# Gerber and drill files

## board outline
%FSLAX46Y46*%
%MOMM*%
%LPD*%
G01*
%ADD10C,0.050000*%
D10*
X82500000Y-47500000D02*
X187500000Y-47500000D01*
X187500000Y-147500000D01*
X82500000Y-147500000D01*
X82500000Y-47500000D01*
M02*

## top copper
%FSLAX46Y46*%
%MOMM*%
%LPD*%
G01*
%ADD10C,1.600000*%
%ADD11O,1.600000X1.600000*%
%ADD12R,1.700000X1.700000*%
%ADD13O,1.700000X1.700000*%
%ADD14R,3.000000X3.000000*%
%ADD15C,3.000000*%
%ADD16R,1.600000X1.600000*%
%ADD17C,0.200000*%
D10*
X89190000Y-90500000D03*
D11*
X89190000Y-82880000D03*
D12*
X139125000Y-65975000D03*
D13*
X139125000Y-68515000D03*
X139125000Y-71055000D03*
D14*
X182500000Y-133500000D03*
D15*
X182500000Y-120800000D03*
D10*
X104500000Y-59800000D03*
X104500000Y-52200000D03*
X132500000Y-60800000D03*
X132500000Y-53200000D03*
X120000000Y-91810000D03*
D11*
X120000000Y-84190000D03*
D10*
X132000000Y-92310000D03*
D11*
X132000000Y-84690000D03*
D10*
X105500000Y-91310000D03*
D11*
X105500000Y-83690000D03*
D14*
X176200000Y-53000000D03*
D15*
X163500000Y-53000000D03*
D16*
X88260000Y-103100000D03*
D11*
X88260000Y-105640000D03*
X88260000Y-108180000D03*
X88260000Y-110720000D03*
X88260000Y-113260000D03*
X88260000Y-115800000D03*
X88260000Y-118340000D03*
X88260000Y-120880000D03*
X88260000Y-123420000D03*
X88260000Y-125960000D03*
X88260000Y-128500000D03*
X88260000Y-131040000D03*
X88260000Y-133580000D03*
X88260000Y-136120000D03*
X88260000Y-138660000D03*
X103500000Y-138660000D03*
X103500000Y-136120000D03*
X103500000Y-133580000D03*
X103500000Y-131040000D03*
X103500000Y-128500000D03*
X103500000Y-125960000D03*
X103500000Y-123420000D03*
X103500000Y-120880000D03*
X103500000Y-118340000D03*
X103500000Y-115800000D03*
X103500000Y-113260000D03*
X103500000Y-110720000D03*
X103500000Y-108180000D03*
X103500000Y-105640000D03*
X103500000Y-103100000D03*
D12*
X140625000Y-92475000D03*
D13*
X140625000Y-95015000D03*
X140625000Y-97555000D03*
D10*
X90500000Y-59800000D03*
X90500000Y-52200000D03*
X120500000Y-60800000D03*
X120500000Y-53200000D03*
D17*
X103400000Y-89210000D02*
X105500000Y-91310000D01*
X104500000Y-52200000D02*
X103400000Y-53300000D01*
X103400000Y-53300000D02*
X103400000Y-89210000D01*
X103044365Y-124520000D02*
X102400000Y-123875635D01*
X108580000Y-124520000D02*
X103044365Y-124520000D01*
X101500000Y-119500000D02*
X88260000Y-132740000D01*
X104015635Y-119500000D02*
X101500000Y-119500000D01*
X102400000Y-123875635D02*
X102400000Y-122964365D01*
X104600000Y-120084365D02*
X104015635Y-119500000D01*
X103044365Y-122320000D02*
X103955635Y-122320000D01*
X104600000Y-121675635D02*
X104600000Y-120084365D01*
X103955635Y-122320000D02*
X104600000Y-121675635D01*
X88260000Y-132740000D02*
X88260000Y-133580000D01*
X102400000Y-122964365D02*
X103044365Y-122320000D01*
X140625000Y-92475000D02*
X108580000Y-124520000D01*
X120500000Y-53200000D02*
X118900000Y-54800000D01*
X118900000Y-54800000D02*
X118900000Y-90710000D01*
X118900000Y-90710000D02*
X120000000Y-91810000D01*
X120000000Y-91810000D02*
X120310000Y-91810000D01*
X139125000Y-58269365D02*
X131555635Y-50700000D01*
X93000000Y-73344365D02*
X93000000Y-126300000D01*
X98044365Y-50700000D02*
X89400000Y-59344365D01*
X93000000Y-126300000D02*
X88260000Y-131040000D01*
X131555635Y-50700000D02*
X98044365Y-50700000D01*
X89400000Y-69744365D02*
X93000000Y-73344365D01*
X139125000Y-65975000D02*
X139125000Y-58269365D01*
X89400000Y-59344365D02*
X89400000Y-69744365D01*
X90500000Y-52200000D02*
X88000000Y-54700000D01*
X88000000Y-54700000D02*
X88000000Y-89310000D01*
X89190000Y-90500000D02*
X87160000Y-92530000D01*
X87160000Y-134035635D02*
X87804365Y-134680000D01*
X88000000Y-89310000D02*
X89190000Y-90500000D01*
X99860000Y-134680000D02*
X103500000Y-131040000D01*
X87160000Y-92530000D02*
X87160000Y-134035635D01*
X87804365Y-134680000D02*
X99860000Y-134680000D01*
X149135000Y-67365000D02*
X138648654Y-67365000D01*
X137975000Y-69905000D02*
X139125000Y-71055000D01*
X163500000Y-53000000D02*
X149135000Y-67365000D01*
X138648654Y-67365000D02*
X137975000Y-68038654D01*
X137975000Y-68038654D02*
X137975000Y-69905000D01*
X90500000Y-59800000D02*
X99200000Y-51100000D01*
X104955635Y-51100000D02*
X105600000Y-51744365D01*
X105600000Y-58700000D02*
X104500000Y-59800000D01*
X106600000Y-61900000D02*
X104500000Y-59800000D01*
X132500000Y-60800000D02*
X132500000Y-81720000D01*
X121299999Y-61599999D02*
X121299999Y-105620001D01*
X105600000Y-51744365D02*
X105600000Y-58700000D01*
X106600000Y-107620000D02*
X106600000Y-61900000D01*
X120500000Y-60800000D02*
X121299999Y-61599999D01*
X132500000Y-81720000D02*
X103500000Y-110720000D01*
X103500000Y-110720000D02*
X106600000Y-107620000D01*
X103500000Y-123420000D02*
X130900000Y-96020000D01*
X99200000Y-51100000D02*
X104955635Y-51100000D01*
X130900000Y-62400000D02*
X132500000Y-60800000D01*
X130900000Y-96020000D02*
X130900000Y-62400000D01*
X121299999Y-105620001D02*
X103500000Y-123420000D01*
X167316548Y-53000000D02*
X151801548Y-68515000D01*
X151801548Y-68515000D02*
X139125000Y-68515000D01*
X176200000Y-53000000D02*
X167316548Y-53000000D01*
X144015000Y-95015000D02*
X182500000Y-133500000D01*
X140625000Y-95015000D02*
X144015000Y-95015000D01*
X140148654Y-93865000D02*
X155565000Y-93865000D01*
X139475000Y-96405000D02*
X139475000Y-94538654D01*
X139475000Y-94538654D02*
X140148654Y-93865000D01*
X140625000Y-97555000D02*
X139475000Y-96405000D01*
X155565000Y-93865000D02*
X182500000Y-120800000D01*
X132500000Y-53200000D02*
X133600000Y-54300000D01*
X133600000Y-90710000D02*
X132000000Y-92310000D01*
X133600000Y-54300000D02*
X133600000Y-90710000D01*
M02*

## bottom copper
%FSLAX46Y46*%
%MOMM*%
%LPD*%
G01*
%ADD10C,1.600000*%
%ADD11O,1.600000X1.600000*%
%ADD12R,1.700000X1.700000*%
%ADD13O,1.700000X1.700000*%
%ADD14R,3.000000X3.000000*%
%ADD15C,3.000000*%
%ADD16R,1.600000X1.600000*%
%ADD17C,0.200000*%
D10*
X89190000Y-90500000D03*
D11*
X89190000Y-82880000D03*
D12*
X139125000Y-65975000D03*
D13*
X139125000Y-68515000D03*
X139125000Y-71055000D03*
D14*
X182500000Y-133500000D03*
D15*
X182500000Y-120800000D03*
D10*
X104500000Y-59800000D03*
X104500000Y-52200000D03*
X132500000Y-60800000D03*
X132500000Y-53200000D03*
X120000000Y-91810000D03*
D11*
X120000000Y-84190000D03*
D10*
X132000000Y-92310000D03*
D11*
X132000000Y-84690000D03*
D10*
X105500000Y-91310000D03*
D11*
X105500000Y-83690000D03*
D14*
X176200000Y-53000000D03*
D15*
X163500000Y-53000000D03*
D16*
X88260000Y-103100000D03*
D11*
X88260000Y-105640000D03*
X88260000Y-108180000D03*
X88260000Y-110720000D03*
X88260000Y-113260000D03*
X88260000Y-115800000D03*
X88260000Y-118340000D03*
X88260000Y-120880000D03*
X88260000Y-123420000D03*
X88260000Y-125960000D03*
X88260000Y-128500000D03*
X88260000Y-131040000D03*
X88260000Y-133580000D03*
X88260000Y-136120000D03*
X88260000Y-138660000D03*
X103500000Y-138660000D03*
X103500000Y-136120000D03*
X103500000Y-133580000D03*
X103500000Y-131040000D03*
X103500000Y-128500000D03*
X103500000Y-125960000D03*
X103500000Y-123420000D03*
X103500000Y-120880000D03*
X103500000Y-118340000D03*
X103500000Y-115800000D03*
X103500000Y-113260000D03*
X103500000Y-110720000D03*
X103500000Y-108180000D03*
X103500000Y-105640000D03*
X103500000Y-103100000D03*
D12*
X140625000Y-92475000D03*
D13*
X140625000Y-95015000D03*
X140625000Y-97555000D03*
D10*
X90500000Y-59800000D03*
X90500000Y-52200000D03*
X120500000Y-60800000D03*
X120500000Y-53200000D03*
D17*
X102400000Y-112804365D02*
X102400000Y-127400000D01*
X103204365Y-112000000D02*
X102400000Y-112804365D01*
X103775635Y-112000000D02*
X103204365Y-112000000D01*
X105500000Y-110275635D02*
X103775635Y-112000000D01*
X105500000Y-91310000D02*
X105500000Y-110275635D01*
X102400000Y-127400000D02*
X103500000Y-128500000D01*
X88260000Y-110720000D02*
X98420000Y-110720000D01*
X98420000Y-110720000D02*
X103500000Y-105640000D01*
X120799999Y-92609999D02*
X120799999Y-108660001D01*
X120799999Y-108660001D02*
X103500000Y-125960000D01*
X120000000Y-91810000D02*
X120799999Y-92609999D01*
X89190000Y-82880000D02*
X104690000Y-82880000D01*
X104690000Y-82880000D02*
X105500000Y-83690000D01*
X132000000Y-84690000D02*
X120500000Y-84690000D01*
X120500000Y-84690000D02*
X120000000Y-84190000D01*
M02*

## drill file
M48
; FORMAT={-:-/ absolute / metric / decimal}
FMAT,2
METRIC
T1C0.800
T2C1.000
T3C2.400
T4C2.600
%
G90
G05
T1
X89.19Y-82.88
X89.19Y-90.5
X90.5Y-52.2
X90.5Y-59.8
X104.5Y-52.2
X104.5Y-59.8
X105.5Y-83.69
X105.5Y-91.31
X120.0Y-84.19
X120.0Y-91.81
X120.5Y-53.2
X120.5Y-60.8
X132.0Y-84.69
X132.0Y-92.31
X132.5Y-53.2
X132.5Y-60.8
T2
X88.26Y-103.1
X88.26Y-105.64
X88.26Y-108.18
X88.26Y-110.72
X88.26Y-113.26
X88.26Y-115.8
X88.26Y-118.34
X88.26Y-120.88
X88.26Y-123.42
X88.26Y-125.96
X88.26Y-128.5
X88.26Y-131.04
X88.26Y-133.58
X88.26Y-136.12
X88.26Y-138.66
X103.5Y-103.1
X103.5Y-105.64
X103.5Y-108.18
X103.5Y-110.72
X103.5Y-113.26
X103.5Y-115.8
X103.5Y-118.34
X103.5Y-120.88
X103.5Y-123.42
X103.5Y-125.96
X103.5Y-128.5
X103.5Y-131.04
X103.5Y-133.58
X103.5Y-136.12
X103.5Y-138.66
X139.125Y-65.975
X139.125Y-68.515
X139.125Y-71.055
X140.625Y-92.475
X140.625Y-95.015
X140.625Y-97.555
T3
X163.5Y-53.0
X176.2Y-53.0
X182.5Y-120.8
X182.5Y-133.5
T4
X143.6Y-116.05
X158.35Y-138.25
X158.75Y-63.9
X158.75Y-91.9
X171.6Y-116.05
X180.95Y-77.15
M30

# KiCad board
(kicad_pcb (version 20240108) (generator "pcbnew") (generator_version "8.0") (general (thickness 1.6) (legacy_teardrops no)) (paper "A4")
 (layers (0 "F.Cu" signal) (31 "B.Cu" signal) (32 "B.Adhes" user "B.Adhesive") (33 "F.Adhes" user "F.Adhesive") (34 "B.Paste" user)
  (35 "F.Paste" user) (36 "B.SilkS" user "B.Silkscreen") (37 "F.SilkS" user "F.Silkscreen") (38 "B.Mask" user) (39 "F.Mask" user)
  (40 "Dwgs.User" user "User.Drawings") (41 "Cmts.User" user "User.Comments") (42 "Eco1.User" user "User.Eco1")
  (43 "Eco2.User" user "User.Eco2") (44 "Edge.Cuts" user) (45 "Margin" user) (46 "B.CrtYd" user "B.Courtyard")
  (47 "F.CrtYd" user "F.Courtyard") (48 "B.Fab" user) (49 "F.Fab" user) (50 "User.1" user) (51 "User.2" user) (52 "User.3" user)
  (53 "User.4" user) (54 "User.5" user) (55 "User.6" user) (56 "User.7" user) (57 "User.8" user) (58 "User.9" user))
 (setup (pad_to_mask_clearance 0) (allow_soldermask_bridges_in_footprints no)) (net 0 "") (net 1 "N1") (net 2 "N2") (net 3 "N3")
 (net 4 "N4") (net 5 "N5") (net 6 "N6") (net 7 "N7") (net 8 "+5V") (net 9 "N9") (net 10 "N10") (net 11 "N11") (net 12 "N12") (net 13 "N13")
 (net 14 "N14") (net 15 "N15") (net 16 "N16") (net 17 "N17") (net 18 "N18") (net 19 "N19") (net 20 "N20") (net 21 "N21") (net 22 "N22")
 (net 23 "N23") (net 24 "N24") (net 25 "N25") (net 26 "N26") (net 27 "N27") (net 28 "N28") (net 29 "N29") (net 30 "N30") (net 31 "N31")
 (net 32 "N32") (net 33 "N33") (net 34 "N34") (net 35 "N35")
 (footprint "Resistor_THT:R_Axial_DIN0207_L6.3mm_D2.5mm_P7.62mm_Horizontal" (layer "F.Cu") (at 89.19 90.5 90)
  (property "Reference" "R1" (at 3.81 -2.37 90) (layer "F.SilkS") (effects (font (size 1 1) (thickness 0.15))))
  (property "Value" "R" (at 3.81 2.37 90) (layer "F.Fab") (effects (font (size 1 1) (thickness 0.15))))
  (pad "1" thru_hole circle (at 0 0 90) (size 1.6 1.6) (drill 0.8) (layers "*.Cu" "*.Mask") (remove_unused_layers no) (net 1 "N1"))
  (pad "2" thru_hole oval (at 7.62 0 90) (size 1.6 1.6) (drill 0.8) (layers "*.Cu" "*.Mask") (remove_unused_layers no) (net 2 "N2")))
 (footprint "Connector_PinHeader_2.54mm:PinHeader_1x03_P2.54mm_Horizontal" (layer "F.Cu") (at 139.125 65.975)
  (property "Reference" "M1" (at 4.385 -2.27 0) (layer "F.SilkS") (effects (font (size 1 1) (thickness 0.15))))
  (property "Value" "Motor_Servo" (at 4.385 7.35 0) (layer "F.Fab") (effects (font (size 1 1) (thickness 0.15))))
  (pad "1" thru_hole rect (at 0 0) (size 1.7 1.7) (drill 1) (layers "*.Cu" "*.Mask") (remove_unused_layers no) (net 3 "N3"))
  (pad "2" thru_hole oval (at 0 2.54) (size 1.7 1.7) (drill 1) (layers "*.Cu" "*.Mask") (remove_unused_layers no) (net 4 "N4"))
  (pad "3" thru_hole oval (at 0 5.08) (size 1.7 1.7) (drill 1) (layers "*.Cu" "*.Mask") (remove_unused_layers no) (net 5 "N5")))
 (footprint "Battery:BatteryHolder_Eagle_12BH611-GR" (layer "F.Cu") (at 182.5 133.5)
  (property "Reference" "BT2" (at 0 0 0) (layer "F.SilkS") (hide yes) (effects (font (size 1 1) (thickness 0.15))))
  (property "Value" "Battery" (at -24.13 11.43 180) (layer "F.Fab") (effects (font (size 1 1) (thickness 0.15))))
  (pad "" np_thru_hole circle (at -38.9 -17.45) (size 2.6 2.6) (drill 2.6) (layers "*.Cu" "*.Mask"))
  (pad "" np_thru_hole circle (at -24.15 4.75) (size 2.6 2.6) (drill 2.6) (layers "*.Cu" "*.Mask"))
  (pad "" np_thru_hole circle (at -10.9 -17.45) (size 2.6 2.6) (drill 2.6) (layers "*.Cu" "*.Mask"))
  (pad "1" thru_hole rect (at 0 0) (size 3 3) (drill 2.4) (layers "*.Cu" "*.Mask") (remove_unused_layers no) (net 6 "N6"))
  (pad "2" thru_hole circle (at 0 -12.7) (size 3 3) (drill 2.4) (layers "*.Cu" "*.Mask") (remove_unused_layers no) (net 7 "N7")))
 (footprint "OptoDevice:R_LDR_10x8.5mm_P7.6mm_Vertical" (layer "F.Cu") (at 104.5 59.8 90)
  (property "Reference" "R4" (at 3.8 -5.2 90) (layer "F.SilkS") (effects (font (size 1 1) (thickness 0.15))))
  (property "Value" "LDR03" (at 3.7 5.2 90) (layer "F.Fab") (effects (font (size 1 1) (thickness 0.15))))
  (pad "1" thru_hole circle (at 0 0 90) (size 1.6 1.6) (drill 0.8) (layers "*.Cu" "*.Mask") (remove_unused_layers no) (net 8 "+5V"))
  (pad "2" thru_hole circle (at 7.6 0 90) (size 1.6 1.6) (drill 0.8) (layers "*.Cu" "*.Mask") (remove_unused_layers no) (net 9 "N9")))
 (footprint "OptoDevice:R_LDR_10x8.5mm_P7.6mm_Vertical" (layer "F.Cu") (at 132.5 60.8 90)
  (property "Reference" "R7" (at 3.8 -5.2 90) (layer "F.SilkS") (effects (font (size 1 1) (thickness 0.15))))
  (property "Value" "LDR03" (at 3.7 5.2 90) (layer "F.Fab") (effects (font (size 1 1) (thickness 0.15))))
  (pad "1" thru_hole circle (at 0 0 90) (size 1.6 1.6) (drill 0.8) (layers "*.Cu" "*.Mask") (remove_unused_layers no) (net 8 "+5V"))
  (pad "2" thru_hole circle (at 7.6 0 90) (size 1.6 1.6) (drill 0.8) (layers "*.Cu" "*.Mask") (remove_unused_layers no) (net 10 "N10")))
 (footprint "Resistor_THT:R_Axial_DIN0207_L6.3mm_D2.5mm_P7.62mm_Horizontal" (layer "F.Cu") (at 120 91.81 90)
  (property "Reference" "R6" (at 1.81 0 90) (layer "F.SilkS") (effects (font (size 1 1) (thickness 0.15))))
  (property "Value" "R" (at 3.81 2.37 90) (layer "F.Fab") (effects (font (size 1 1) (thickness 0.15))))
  (pad "1" thru_hole circle (at 0 0 90) (size 1.6 1.6) (drill 0.8) (layers "*.Cu" "*.Mask") (remove_unused_layers no) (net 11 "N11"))
  (pad "2" thru_hole oval (at 7.62 0 90) (size 1.6 1.6) (drill 0.8) (layers "*.Cu" "*.Mask") (remove_unused_layers no) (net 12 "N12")))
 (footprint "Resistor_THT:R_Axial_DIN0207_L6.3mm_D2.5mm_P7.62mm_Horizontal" (layer "F.Cu") (at 132 92.31 90)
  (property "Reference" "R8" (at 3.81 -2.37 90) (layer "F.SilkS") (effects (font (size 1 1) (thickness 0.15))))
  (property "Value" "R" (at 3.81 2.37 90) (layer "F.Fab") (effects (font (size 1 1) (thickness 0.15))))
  (pad "1" thru_hole circle (at 0 0 90) (size 1.6 1.6) (drill 0.8) (layers "*.Cu" "*.Mask") (remove_unused_layers no) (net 10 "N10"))
  (pad "2" thru_hole oval (at 7.62 0 90) (size 1.6 1.6) (drill 0.8) (layers "*.Cu" "*.Mask") (remove_unused_layers no) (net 12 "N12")))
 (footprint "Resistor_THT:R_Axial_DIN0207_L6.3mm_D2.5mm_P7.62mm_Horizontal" (layer "F.Cu") (at 105.5 91.31 90)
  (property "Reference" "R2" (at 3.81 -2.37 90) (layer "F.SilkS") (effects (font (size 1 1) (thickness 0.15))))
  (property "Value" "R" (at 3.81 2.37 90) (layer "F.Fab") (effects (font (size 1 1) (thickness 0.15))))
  (pad "1" thru_hole circle (at 0 0 90) (size 1.6 1.6) (drill 0.8) (layers "*.Cu" "*.Mask") (remove_unused_layers no) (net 9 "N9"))
  (pad "2" thru_hole oval (at 7.62 0 90) (size 1.6 1.6) (drill 0.8) (layers "*.Cu" "*.Mask") (remove_unused_layers no) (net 2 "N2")))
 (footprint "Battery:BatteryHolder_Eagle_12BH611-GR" (layer "F.Cu") (at 176.2 53 90)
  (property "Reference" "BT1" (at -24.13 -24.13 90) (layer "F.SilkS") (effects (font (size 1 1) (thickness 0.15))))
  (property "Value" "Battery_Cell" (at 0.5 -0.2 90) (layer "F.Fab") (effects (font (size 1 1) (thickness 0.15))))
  (pad "" np_thru_hole circle (at -38.9 -17.45 90) (size 2.6 2.6) (drill 2.6) (layers "*.Cu" "*.Mask"))
  (pad "" np_thru_hole circle (at -24.15 4.75 90) (size 2.6 2.6) (drill 2.6) (layers "*.Cu" "*.Mask"))
  (pad "" np_thru_hole circle (at -10.9 -17.45 90) (size 2.6 2.6) (drill 2.6) (layers "*.Cu" "*.Mask"))
  (pad "1" thru_hole rect (at 0 0 90) (size 3 3) (drill 2.4) (layers "*.Cu" "*.Mask") (remove_unused_layers no) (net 4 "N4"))
  (pad "2" thru_hole circle (at 0 -12.7 90) (size 3 3) (drill 2.4) (layers "*.Cu" "*.Mask") (remove_unused_layers no) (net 5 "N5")))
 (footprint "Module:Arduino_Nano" (layer "F.Cu") (at 88.26 103.1)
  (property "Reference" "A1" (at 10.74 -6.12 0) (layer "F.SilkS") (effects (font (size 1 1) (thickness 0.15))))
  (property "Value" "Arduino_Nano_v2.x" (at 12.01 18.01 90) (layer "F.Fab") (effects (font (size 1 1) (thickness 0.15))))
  (pad "1" thru_hole rect (at 0 0) (size 1.6 1.6) (drill 1) (layers "*.Cu" "*.Mask") (remove_unused_layers no) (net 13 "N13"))
  (pad "2" thru_hole oval (at 0 2.54) (size 1.6 1.6) (drill 1) (layers "*.Cu" "*.Mask") (remove_unused_layers no) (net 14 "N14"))
  (pad "3" thru_hole oval (at 0 5.08) (size 1.6 1.6) (drill 1) (layers "*.Cu" "*.Mask") (remove_unused_layers no) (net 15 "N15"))
  (pad "4" thru_hole oval (at 0 7.62) (size 1.6 1.6) (drill 1) (layers "*.Cu" "*.Mask") (remove_unused_layers no) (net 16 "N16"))
  (pad "5" thru_hole oval (at 0 10.16) (size 1.6 1.6) (drill 1) (layers "*.Cu" "*.Mask") (remove_unused_layers no) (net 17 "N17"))
  (pad "6" thru_hole oval (at 0 12.7) (size 1.6 1.6) (drill 1) (layers "*.Cu" "*.Mask") (remove_unused_layers no) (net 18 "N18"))
  (pad "7" thru_hole oval (at 0 15.24) (size 1.6 1.6) (drill 1) (layers "*.Cu" "*.Mask") (remove_unused_layers no) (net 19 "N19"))
  (pad "8" thru_hole oval (at 0 17.78) (size 1.6 1.6) (drill 1) (layers "*.Cu" "*.Mask") (remove_unused_layers no) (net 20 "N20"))
  (pad "9" thru_hole oval (at 0 20.32) (size 1.6 1.6) (drill 1) (layers "*.Cu" "*.Mask") (remove_unused_layers no) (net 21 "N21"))
  (pad "10" thru_hole oval (at 0 22.86) (size 1.6 1.6) (drill 1) (layers "*.Cu" "*.Mask") (remove_unused_layers no) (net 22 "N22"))
  (pad "11" thru_hole oval (at 0 25.4) (size 1.6 1.6) (drill 1) (layers "*.Cu" "*.Mask") (remove_unused_layers no) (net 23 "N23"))
  (pad "12" thru_hole oval (at 0 27.94) (size 1.6 1.6) (drill 1) (layers "*.Cu" "*.Mask") (remove_unused_layers no) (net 3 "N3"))
  (pad "13" thru_hole oval (at 0 30.48) (size 1.6 1.6) (drill 1) (layers "*.Cu" "*.Mask") (remove_unused_layers no) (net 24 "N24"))
  (pad "14" thru_hole oval (at 0 33.02) (size 1.6 1.6) (drill 1) (layers "*.Cu" "*.Mask") (remove_unused_layers no) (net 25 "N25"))
  (pad "15" thru_hole oval (at 0 35.56) (size 1.6 1.6) (drill 1) (layers "*.Cu" "*.Mask") (remove_unused_layers no) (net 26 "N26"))
  (pad "16" thru_hole oval (at 15.24 35.56) (size 1.6 1.6) (drill 1) (layers "*.Cu" "*.Mask") (remove_unused_layers no) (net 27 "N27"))
  (pad "17" thru_hole oval (at 15.24 33.02) (size 1.6 1.6) (drill 1) (layers "*.Cu" "*.Mask") (remove_unused_layers no) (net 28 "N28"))
  (pad "18" thru_hole oval (at 15.24 30.48) (size 1.6 1.6) (drill 1) (layers "*.Cu" "*.Mask") (remove_unused_layers no) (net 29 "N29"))
  (pad "19" thru_hole oval (at 15.24 27.94) (size 1.6 1.6) (drill 1) (layers "*.Cu" "*.Mask") (remove_unused_layers no) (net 1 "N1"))
  (pad "20" thru_hole oval (at 15.24 25.4) (size 1.6 1.6) (drill 1) (layers "*.Cu" "*.Mask") (remove_unused_layers no) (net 9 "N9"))
  (pad "21" thru_hole oval (at 15.24 22.86) (size 1.6 1.6) (drill 1) (layers "*.Cu" "*.Mask") (remove_unused_layers no) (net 11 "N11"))
  (pad "22" thru_hole oval (at 15.24 20.32) (size 1.6 1.6) (drill 1) (layers "*.Cu" "*.Mask") (remove_unused_layers no) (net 8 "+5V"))
  (pad "23" thru_hole oval (at 15.24 17.78) (size 1.6 1.6) (drill 1) (layers "*.Cu" "*.Mask") (remove_unused_layers no) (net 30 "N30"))
  (pad "24" thru_hole oval (at 15.24 15.24) (size 1.6 1.6) (drill 1) (layers "*.Cu" "*.Mask") (remove_unused_layers no) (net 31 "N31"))
  (pad "25" thru_hole oval (at 15.24 12.7) (size 1.6 1.6) (drill 1) (layers "*.Cu" "*.Mask") (remove_unused_layers no) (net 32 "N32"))
  (pad "26" thru_hole oval (at 15.24 10.16) (size 1.6 1.6) (drill 1) (layers "*.Cu" "*.Mask") (remove_unused_layers no) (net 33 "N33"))
  (pad "27" thru_hole oval (at 15.24 7.62) (size 1.6 1.6) (drill 1) (layers "*.Cu" "*.Mask") (remove_unused_layers no) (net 8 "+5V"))
  (pad "28" thru_hole oval (at 15.24 5.08) (size 1.6 1.6) (drill 1) (layers "*.Cu" "*.Mask") (remove_unused_layers no) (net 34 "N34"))
  (pad "29" thru_hole oval (at 15.24 2.54) (size 1.6 1.6) (drill 1) (layers "*.Cu" "*.Mask") (remove_unused_layers no) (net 16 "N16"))
  (pad "30" thru_hole oval (at 15.24 0) (size 1.6 1.6) (drill 1) (layers "*.Cu" "*.Mask") (remove_unused_layers no) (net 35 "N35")))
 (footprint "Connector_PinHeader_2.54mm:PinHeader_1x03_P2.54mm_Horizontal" (layer "F.Cu") (at 140.625 92.475)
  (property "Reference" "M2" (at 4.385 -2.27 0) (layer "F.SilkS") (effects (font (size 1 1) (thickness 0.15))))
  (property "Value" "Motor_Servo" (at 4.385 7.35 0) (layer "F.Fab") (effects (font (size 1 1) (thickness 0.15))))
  (pad "1" thru_hole rect (at 0 0) (size 1.7 1.7) (drill 1) (layers "*.Cu" "*.Mask") (remove_unused_layers no) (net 24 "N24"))
  (pad "2" thru_hole oval (at 0 2.54) (size 1.7 1.7) (drill 1) (layers "*.Cu" "*.Mask") (remove_unused_layers no) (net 6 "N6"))
  (pad "3" thru_hole oval (at 0 5.08) (size 1.7 1.7) (drill 1) (layers "*.Cu" "*.Mask") (remove_unused_layers no) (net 7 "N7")))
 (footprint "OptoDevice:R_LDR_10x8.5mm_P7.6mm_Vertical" (layer "F.Cu") (at 90.5 59.8 90)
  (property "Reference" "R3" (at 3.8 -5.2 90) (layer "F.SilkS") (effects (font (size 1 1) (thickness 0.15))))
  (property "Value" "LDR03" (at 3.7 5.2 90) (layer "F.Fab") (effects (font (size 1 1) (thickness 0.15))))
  (pad "1" thru_hole circle (at 0 0 90) (size 1.6 1.6) (drill 0.8) (layers "*.Cu" "*.Mask") (remove_unused_layers no) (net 8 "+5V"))
  (pad "2" thru_hole circle (at 7.6 0 90) (size 1.6 1.6) (drill 0.8) (layers "*.Cu" "*.Mask") (remove_unused_layers no) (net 1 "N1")))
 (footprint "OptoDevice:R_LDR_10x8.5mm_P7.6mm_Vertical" (layer "F.Cu") (at 120.5 60.8 90)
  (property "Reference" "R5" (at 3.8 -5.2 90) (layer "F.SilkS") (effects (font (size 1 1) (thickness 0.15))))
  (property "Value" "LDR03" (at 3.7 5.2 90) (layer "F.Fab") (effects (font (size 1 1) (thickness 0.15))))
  (pad "1" thru_hole circle (at 0 0 90) (size 1.6 1.6) (drill 0.8) (layers "*.Cu" "*.Mask") (remove_unused_layers no) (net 8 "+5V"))
  (pad "2" thru_hole circle (at 7.6 0 90) (size 1.6 1.6) (drill 0.8) (layers "*.Cu" "*.Mask") (remove_unused_layers no) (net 11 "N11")))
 (gr_rect (start 82.5 47.5) (end 187.5 147.5) (stroke (width 0.05) (type default)) (fill none) (layer "Edge.Cuts"))
 (segment (start 103.4 89.21) (end 105.5 91.31) (width 0.2) (layer "F.Cu") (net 9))
 (segment (start 104.5 52.2) (end 103.4 53.3) (width 0.2) (layer "F.Cu") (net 9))
 (segment (start 103.4 53.3) (end 103.4 89.21) (width 0.2) (layer "F.Cu") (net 9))
 (segment (start 102.4 112.804365) (end 102.4 127.4) (width 0.2) (layer "B.Cu") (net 9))
 (segment (start 103.204365 112) (end 102.4 112.804365) (width 0.2) (layer "B.Cu") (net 9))
 (segment (start 103.775635 112) (end 103.204365 112) (width 0.2) (layer "B.Cu") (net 9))
 (segment (start 105.5 110.275635) (end 103.775635 112) (width 0.2) (layer "B.Cu") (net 9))
 (segment (start 105.5 91.31) (end 105.5 110.275635) (width 0.2) (layer "B.Cu") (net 9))
 (segment (start 102.4 127.4) (end 103.5 128.5) (width 0.2) (layer "B.Cu") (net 9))
 (segment (start 88.26 110.72) (end 98.42 110.72) (width 0.2) (layer "B.Cu") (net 16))
 (segment (start 98.42 110.72) (end 103.5 105.64) (width 0.2) (layer "B.Cu") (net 16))
 (segment (start 103.044365 124.52) (end 102.4 123.875635) (width 0.2) (layer "F.Cu") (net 24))
 (segment (start 108.58 124.52) (end 103.044365 124.52) (width 0.2) (layer "F.Cu") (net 24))
 (segment (start 101.5 119.5) (end 88.26 132.74) (width 0.2) (layer "F.Cu") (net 24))
 (segment (start 104.015635 119.5) (end 101.5 119.5) (width 0.2) (layer "F.Cu") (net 24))
 (segment (start 102.4 123.875635) (end 102.4 122.964365) (width 0.2) (layer "F.Cu") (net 24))
 (segment (start 104.6 120.084365) (end 104.015635 119.5) (width 0.2) (layer "F.Cu") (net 24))
 (segment (start 103.044365 122.32) (end 103.955635 122.32) (width 0.2) (layer "F.Cu") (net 24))
 (segment (start 104.6 121.675635) (end 104.6 120.084365) (width 0.2) (layer "F.Cu") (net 24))
 (segment (start 103.955635 122.32) (end 104.6 121.675635) (width 0.2) (layer "F.Cu") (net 24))
 (segment (start 88.26 132.74) (end 88.26 133.58) (width 0.2) (layer "F.Cu") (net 24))
 (segment (start 102.4 122.964365) (end 103.044365 122.32) (width 0.2) (layer "F.Cu") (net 24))
 (segment (start 140.625 92.475) (end 108.58 124.52) (width 0.2) (layer "F.Cu") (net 24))
 (segment (start 120.5 53.2) (end 118.9 54.8) (width 0.2) (layer "F.Cu") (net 11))
 (segment (start 118.9 54.8) (end 118.9 90.71) (width 0.2) (layer "F.Cu") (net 11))
 (segment (start 118.9 90.71) (end 120 91.81) (width 0.2) (layer "F.Cu") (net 11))
 (segment (start 120 91.81) (end 120.31 91.81) (width 0.2) (layer "F.Cu") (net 11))
 (segment (start 120.799999 92.609999) (end 120.799999 108.660001) (width 0.2) (layer "B.Cu") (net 11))
 (segment (start 120.799999 108.660001) (end 103.5 125.96) (width 0.2) (layer "B.Cu") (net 11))
 (segment (start 120 91.81) (end 120.799999 92.609999) (width 0.2) (layer "B.Cu") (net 11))
 (segment (start 139.125 58.269365) (end 131.555635 50.7) (width 0.2) (layer "F.Cu") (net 3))
 (segment (start 93 73.344365) (end 93 126.3) (width 0.2) (layer "F.Cu") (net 3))
 (segment (start 98.044365 50.7) (end 89.4 59.344365) (width 0.2) (layer "F.Cu") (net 3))
 (segment (start 93 126.3) (end 88.26 131.04) (width 0.2) (layer "F.Cu") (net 3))
 (segment (start 131.555635 50.7) (end 98.044365 50.7) (width 0.2) (layer "F.Cu") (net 3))
 (segment (start 89.4 69.744365) (end 93 73.344365) (width 0.2) (layer "F.Cu") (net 3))
 (segment (start 139.125 65.975) (end 139.125 58.269365) (width 0.2) (layer "F.Cu") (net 3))
 (segment (start 89.4 59.344365) (end 89.4 69.744365) (width 0.2) (layer "F.Cu") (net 3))
 (segment (start 90.5 52.2) (end 88 54.7) (width 0.2) (layer "F.Cu") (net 1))
 (segment (start 88 54.7) (end 88 89.31) (width 0.2) (layer "F.Cu") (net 1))
 (segment (start 89.19 90.5) (end 87.16 92.53) (width 0.2) (layer "F.Cu") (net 1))
 (segment (start 87.16 134.035635) (end 87.804365 134.68) (width 0.2) (layer "F.Cu") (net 1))
 (segment (start 88 89.31) (end 89.19 90.5) (width 0.2) (layer "F.Cu") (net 1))
 (segment (start 99.86 134.68) (end 103.5 131.04) (width 0.2) (layer "F.Cu") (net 1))
 (segment (start 87.16 92.53) (end 87.16 134.035635) (width 0.2) (layer "F.Cu") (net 1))
 (segment (start 87.804365 134.68) (end 99.86 134.68) (width 0.2) (layer "F.Cu") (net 1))
 (segment (start 149.135 67.365) (end 138.648654 67.365) (width 0.2) (layer "F.Cu") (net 5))
 (segment (start 137.975 69.905) (end 139.125 71.055) (width 0.2) (layer "F.Cu") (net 5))
 (segment (start 163.5 53) (end 149.135 67.365) (width 0.2) (layer "F.Cu") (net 5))
 (segment (start 138.648654 67.365) (end 137.975 68.038654) (width 0.2) (layer "F.Cu") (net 5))
 (segment (start 137.975 68.038654) (end 137.975 69.905) (width 0.2) (layer "F.Cu") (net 5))
 (segment (start 90.5 59.8) (end 99.2 51.1) (width 0.2) (layer "F.Cu") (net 8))
 (segment (start 104.955635 51.1) (end 105.6 51.744365) (width 0.2) (layer "F.Cu") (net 8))
 (segment (start 105.6 58.7) (end 104.5 59.8) (width 0.2) (layer "F.Cu") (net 8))
 (segment (start 106.6 61.9) (end 104.5 59.8) (width 0.2) (layer "F.Cu") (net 8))
 (segment (start 132.5 60.8) (end 132.5 81.72) (width 0.2) (layer "F.Cu") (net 8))
 (segment (start 121.299999 61.599999) (end 121.299999 105.620001) (width 0.2) (layer "F.Cu") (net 8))
 (segment (start 105.6 51.744365) (end 105.6 58.7) (width 0.2) (layer "F.Cu") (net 8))
 (segment (start 106.6 107.62) (end 106.6 61.9) (width 0.2) (layer "F.Cu") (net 8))
 (segment (start 120.5 60.8) (end 121.299999 61.599999) (width 0.2) (layer "F.Cu") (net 8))
 (segment (start 132.5 81.72) (end 103.5 110.72) (width 0.2) (layer "F.Cu") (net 8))
 (segment (start 103.5 110.72) (end 106.6 107.62) (width 0.2) (layer "F.Cu") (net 8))
 (segment (start 103.5 123.42) (end 130.9 96.02) (width 0.2) (layer "F.Cu") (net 8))
 (segment (start 99.2 51.1) (end 104.955635 51.1) (width 0.2) (layer "F.Cu") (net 8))
 (segment (start 130.9 62.4) (end 132.5 60.8) (width 0.2) (layer "F.Cu") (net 8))
 (segment (start 130.9 96.02) (end 130.9 62.4) (width 0.2) (layer "F.Cu") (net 8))
 (segment (start 121.299999 105.620001) (end 103.5 123.42) (width 0.2) (layer "F.Cu") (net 8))
 (segment (start 167.316548 53) (end 151.801548 68.515) (width 0.2) (layer "F.Cu") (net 4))
 (segment (start 151.801548 68.515) (end 139.125 68.515) (width 0.2) (layer "F.Cu") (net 4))
 (segment (start 176.2 53) (end 167.316548 53) (width 0.2) (layer "F.Cu") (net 4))
 (segment (start 144.015 95.015) (end 182.5 133.5) (width 0.2) (layer "F.Cu") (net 6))
 (segment (start 140.625 95.015) (end 144.015 95.015) (width 0.2) (layer "F.Cu") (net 6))
 (segment (start 140.148654 93.865) (end 155.565 93.865) (width 0.2) (layer "F.Cu") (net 7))
 (segment (start 139.475 96.405) (end 139.475 94.538654) (width 0.2) (layer "F.Cu") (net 7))
 (segment (start 139.475 94.538654) (end 140.148654 93.865) (width 0.2) (layer "F.Cu") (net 7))
 (segment (start 140.625 97.555) (end 139.475 96.405) (width 0.2) (layer "F.Cu") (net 7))
 (segment (start 155.565 93.865) (end 182.5 120.8) (width 0.2) (layer "F.Cu") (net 7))
 (segment (start 89.19 82.88) (end 104.69 82.88) (width 0.2) (layer "B.Cu") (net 2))
 (segment (start 104.69 82.88) (end 105.5 83.69) (width 0.2) (layer "B.Cu") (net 2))
 (segment (start 132 84.69) (end 120.5 84.69) (width 0.2) (layer "B.Cu") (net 12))
 (segment (start 120.5 84.69) (end 120 84.19) (width 0.2) (layer "B.Cu") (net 12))
 (segment (start 132.5 53.2) (end 133.6 54.3) (width 0.2) (layer "F.Cu") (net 10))
 (segment (start 133.6 90.71) (end 132 92.31) (width 0.2) (layer "F.Cu") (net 10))
 (segment (start 133.6 54.3) (end 133.6 90.71) (width 0.2) (layer "F.Cu") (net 10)))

